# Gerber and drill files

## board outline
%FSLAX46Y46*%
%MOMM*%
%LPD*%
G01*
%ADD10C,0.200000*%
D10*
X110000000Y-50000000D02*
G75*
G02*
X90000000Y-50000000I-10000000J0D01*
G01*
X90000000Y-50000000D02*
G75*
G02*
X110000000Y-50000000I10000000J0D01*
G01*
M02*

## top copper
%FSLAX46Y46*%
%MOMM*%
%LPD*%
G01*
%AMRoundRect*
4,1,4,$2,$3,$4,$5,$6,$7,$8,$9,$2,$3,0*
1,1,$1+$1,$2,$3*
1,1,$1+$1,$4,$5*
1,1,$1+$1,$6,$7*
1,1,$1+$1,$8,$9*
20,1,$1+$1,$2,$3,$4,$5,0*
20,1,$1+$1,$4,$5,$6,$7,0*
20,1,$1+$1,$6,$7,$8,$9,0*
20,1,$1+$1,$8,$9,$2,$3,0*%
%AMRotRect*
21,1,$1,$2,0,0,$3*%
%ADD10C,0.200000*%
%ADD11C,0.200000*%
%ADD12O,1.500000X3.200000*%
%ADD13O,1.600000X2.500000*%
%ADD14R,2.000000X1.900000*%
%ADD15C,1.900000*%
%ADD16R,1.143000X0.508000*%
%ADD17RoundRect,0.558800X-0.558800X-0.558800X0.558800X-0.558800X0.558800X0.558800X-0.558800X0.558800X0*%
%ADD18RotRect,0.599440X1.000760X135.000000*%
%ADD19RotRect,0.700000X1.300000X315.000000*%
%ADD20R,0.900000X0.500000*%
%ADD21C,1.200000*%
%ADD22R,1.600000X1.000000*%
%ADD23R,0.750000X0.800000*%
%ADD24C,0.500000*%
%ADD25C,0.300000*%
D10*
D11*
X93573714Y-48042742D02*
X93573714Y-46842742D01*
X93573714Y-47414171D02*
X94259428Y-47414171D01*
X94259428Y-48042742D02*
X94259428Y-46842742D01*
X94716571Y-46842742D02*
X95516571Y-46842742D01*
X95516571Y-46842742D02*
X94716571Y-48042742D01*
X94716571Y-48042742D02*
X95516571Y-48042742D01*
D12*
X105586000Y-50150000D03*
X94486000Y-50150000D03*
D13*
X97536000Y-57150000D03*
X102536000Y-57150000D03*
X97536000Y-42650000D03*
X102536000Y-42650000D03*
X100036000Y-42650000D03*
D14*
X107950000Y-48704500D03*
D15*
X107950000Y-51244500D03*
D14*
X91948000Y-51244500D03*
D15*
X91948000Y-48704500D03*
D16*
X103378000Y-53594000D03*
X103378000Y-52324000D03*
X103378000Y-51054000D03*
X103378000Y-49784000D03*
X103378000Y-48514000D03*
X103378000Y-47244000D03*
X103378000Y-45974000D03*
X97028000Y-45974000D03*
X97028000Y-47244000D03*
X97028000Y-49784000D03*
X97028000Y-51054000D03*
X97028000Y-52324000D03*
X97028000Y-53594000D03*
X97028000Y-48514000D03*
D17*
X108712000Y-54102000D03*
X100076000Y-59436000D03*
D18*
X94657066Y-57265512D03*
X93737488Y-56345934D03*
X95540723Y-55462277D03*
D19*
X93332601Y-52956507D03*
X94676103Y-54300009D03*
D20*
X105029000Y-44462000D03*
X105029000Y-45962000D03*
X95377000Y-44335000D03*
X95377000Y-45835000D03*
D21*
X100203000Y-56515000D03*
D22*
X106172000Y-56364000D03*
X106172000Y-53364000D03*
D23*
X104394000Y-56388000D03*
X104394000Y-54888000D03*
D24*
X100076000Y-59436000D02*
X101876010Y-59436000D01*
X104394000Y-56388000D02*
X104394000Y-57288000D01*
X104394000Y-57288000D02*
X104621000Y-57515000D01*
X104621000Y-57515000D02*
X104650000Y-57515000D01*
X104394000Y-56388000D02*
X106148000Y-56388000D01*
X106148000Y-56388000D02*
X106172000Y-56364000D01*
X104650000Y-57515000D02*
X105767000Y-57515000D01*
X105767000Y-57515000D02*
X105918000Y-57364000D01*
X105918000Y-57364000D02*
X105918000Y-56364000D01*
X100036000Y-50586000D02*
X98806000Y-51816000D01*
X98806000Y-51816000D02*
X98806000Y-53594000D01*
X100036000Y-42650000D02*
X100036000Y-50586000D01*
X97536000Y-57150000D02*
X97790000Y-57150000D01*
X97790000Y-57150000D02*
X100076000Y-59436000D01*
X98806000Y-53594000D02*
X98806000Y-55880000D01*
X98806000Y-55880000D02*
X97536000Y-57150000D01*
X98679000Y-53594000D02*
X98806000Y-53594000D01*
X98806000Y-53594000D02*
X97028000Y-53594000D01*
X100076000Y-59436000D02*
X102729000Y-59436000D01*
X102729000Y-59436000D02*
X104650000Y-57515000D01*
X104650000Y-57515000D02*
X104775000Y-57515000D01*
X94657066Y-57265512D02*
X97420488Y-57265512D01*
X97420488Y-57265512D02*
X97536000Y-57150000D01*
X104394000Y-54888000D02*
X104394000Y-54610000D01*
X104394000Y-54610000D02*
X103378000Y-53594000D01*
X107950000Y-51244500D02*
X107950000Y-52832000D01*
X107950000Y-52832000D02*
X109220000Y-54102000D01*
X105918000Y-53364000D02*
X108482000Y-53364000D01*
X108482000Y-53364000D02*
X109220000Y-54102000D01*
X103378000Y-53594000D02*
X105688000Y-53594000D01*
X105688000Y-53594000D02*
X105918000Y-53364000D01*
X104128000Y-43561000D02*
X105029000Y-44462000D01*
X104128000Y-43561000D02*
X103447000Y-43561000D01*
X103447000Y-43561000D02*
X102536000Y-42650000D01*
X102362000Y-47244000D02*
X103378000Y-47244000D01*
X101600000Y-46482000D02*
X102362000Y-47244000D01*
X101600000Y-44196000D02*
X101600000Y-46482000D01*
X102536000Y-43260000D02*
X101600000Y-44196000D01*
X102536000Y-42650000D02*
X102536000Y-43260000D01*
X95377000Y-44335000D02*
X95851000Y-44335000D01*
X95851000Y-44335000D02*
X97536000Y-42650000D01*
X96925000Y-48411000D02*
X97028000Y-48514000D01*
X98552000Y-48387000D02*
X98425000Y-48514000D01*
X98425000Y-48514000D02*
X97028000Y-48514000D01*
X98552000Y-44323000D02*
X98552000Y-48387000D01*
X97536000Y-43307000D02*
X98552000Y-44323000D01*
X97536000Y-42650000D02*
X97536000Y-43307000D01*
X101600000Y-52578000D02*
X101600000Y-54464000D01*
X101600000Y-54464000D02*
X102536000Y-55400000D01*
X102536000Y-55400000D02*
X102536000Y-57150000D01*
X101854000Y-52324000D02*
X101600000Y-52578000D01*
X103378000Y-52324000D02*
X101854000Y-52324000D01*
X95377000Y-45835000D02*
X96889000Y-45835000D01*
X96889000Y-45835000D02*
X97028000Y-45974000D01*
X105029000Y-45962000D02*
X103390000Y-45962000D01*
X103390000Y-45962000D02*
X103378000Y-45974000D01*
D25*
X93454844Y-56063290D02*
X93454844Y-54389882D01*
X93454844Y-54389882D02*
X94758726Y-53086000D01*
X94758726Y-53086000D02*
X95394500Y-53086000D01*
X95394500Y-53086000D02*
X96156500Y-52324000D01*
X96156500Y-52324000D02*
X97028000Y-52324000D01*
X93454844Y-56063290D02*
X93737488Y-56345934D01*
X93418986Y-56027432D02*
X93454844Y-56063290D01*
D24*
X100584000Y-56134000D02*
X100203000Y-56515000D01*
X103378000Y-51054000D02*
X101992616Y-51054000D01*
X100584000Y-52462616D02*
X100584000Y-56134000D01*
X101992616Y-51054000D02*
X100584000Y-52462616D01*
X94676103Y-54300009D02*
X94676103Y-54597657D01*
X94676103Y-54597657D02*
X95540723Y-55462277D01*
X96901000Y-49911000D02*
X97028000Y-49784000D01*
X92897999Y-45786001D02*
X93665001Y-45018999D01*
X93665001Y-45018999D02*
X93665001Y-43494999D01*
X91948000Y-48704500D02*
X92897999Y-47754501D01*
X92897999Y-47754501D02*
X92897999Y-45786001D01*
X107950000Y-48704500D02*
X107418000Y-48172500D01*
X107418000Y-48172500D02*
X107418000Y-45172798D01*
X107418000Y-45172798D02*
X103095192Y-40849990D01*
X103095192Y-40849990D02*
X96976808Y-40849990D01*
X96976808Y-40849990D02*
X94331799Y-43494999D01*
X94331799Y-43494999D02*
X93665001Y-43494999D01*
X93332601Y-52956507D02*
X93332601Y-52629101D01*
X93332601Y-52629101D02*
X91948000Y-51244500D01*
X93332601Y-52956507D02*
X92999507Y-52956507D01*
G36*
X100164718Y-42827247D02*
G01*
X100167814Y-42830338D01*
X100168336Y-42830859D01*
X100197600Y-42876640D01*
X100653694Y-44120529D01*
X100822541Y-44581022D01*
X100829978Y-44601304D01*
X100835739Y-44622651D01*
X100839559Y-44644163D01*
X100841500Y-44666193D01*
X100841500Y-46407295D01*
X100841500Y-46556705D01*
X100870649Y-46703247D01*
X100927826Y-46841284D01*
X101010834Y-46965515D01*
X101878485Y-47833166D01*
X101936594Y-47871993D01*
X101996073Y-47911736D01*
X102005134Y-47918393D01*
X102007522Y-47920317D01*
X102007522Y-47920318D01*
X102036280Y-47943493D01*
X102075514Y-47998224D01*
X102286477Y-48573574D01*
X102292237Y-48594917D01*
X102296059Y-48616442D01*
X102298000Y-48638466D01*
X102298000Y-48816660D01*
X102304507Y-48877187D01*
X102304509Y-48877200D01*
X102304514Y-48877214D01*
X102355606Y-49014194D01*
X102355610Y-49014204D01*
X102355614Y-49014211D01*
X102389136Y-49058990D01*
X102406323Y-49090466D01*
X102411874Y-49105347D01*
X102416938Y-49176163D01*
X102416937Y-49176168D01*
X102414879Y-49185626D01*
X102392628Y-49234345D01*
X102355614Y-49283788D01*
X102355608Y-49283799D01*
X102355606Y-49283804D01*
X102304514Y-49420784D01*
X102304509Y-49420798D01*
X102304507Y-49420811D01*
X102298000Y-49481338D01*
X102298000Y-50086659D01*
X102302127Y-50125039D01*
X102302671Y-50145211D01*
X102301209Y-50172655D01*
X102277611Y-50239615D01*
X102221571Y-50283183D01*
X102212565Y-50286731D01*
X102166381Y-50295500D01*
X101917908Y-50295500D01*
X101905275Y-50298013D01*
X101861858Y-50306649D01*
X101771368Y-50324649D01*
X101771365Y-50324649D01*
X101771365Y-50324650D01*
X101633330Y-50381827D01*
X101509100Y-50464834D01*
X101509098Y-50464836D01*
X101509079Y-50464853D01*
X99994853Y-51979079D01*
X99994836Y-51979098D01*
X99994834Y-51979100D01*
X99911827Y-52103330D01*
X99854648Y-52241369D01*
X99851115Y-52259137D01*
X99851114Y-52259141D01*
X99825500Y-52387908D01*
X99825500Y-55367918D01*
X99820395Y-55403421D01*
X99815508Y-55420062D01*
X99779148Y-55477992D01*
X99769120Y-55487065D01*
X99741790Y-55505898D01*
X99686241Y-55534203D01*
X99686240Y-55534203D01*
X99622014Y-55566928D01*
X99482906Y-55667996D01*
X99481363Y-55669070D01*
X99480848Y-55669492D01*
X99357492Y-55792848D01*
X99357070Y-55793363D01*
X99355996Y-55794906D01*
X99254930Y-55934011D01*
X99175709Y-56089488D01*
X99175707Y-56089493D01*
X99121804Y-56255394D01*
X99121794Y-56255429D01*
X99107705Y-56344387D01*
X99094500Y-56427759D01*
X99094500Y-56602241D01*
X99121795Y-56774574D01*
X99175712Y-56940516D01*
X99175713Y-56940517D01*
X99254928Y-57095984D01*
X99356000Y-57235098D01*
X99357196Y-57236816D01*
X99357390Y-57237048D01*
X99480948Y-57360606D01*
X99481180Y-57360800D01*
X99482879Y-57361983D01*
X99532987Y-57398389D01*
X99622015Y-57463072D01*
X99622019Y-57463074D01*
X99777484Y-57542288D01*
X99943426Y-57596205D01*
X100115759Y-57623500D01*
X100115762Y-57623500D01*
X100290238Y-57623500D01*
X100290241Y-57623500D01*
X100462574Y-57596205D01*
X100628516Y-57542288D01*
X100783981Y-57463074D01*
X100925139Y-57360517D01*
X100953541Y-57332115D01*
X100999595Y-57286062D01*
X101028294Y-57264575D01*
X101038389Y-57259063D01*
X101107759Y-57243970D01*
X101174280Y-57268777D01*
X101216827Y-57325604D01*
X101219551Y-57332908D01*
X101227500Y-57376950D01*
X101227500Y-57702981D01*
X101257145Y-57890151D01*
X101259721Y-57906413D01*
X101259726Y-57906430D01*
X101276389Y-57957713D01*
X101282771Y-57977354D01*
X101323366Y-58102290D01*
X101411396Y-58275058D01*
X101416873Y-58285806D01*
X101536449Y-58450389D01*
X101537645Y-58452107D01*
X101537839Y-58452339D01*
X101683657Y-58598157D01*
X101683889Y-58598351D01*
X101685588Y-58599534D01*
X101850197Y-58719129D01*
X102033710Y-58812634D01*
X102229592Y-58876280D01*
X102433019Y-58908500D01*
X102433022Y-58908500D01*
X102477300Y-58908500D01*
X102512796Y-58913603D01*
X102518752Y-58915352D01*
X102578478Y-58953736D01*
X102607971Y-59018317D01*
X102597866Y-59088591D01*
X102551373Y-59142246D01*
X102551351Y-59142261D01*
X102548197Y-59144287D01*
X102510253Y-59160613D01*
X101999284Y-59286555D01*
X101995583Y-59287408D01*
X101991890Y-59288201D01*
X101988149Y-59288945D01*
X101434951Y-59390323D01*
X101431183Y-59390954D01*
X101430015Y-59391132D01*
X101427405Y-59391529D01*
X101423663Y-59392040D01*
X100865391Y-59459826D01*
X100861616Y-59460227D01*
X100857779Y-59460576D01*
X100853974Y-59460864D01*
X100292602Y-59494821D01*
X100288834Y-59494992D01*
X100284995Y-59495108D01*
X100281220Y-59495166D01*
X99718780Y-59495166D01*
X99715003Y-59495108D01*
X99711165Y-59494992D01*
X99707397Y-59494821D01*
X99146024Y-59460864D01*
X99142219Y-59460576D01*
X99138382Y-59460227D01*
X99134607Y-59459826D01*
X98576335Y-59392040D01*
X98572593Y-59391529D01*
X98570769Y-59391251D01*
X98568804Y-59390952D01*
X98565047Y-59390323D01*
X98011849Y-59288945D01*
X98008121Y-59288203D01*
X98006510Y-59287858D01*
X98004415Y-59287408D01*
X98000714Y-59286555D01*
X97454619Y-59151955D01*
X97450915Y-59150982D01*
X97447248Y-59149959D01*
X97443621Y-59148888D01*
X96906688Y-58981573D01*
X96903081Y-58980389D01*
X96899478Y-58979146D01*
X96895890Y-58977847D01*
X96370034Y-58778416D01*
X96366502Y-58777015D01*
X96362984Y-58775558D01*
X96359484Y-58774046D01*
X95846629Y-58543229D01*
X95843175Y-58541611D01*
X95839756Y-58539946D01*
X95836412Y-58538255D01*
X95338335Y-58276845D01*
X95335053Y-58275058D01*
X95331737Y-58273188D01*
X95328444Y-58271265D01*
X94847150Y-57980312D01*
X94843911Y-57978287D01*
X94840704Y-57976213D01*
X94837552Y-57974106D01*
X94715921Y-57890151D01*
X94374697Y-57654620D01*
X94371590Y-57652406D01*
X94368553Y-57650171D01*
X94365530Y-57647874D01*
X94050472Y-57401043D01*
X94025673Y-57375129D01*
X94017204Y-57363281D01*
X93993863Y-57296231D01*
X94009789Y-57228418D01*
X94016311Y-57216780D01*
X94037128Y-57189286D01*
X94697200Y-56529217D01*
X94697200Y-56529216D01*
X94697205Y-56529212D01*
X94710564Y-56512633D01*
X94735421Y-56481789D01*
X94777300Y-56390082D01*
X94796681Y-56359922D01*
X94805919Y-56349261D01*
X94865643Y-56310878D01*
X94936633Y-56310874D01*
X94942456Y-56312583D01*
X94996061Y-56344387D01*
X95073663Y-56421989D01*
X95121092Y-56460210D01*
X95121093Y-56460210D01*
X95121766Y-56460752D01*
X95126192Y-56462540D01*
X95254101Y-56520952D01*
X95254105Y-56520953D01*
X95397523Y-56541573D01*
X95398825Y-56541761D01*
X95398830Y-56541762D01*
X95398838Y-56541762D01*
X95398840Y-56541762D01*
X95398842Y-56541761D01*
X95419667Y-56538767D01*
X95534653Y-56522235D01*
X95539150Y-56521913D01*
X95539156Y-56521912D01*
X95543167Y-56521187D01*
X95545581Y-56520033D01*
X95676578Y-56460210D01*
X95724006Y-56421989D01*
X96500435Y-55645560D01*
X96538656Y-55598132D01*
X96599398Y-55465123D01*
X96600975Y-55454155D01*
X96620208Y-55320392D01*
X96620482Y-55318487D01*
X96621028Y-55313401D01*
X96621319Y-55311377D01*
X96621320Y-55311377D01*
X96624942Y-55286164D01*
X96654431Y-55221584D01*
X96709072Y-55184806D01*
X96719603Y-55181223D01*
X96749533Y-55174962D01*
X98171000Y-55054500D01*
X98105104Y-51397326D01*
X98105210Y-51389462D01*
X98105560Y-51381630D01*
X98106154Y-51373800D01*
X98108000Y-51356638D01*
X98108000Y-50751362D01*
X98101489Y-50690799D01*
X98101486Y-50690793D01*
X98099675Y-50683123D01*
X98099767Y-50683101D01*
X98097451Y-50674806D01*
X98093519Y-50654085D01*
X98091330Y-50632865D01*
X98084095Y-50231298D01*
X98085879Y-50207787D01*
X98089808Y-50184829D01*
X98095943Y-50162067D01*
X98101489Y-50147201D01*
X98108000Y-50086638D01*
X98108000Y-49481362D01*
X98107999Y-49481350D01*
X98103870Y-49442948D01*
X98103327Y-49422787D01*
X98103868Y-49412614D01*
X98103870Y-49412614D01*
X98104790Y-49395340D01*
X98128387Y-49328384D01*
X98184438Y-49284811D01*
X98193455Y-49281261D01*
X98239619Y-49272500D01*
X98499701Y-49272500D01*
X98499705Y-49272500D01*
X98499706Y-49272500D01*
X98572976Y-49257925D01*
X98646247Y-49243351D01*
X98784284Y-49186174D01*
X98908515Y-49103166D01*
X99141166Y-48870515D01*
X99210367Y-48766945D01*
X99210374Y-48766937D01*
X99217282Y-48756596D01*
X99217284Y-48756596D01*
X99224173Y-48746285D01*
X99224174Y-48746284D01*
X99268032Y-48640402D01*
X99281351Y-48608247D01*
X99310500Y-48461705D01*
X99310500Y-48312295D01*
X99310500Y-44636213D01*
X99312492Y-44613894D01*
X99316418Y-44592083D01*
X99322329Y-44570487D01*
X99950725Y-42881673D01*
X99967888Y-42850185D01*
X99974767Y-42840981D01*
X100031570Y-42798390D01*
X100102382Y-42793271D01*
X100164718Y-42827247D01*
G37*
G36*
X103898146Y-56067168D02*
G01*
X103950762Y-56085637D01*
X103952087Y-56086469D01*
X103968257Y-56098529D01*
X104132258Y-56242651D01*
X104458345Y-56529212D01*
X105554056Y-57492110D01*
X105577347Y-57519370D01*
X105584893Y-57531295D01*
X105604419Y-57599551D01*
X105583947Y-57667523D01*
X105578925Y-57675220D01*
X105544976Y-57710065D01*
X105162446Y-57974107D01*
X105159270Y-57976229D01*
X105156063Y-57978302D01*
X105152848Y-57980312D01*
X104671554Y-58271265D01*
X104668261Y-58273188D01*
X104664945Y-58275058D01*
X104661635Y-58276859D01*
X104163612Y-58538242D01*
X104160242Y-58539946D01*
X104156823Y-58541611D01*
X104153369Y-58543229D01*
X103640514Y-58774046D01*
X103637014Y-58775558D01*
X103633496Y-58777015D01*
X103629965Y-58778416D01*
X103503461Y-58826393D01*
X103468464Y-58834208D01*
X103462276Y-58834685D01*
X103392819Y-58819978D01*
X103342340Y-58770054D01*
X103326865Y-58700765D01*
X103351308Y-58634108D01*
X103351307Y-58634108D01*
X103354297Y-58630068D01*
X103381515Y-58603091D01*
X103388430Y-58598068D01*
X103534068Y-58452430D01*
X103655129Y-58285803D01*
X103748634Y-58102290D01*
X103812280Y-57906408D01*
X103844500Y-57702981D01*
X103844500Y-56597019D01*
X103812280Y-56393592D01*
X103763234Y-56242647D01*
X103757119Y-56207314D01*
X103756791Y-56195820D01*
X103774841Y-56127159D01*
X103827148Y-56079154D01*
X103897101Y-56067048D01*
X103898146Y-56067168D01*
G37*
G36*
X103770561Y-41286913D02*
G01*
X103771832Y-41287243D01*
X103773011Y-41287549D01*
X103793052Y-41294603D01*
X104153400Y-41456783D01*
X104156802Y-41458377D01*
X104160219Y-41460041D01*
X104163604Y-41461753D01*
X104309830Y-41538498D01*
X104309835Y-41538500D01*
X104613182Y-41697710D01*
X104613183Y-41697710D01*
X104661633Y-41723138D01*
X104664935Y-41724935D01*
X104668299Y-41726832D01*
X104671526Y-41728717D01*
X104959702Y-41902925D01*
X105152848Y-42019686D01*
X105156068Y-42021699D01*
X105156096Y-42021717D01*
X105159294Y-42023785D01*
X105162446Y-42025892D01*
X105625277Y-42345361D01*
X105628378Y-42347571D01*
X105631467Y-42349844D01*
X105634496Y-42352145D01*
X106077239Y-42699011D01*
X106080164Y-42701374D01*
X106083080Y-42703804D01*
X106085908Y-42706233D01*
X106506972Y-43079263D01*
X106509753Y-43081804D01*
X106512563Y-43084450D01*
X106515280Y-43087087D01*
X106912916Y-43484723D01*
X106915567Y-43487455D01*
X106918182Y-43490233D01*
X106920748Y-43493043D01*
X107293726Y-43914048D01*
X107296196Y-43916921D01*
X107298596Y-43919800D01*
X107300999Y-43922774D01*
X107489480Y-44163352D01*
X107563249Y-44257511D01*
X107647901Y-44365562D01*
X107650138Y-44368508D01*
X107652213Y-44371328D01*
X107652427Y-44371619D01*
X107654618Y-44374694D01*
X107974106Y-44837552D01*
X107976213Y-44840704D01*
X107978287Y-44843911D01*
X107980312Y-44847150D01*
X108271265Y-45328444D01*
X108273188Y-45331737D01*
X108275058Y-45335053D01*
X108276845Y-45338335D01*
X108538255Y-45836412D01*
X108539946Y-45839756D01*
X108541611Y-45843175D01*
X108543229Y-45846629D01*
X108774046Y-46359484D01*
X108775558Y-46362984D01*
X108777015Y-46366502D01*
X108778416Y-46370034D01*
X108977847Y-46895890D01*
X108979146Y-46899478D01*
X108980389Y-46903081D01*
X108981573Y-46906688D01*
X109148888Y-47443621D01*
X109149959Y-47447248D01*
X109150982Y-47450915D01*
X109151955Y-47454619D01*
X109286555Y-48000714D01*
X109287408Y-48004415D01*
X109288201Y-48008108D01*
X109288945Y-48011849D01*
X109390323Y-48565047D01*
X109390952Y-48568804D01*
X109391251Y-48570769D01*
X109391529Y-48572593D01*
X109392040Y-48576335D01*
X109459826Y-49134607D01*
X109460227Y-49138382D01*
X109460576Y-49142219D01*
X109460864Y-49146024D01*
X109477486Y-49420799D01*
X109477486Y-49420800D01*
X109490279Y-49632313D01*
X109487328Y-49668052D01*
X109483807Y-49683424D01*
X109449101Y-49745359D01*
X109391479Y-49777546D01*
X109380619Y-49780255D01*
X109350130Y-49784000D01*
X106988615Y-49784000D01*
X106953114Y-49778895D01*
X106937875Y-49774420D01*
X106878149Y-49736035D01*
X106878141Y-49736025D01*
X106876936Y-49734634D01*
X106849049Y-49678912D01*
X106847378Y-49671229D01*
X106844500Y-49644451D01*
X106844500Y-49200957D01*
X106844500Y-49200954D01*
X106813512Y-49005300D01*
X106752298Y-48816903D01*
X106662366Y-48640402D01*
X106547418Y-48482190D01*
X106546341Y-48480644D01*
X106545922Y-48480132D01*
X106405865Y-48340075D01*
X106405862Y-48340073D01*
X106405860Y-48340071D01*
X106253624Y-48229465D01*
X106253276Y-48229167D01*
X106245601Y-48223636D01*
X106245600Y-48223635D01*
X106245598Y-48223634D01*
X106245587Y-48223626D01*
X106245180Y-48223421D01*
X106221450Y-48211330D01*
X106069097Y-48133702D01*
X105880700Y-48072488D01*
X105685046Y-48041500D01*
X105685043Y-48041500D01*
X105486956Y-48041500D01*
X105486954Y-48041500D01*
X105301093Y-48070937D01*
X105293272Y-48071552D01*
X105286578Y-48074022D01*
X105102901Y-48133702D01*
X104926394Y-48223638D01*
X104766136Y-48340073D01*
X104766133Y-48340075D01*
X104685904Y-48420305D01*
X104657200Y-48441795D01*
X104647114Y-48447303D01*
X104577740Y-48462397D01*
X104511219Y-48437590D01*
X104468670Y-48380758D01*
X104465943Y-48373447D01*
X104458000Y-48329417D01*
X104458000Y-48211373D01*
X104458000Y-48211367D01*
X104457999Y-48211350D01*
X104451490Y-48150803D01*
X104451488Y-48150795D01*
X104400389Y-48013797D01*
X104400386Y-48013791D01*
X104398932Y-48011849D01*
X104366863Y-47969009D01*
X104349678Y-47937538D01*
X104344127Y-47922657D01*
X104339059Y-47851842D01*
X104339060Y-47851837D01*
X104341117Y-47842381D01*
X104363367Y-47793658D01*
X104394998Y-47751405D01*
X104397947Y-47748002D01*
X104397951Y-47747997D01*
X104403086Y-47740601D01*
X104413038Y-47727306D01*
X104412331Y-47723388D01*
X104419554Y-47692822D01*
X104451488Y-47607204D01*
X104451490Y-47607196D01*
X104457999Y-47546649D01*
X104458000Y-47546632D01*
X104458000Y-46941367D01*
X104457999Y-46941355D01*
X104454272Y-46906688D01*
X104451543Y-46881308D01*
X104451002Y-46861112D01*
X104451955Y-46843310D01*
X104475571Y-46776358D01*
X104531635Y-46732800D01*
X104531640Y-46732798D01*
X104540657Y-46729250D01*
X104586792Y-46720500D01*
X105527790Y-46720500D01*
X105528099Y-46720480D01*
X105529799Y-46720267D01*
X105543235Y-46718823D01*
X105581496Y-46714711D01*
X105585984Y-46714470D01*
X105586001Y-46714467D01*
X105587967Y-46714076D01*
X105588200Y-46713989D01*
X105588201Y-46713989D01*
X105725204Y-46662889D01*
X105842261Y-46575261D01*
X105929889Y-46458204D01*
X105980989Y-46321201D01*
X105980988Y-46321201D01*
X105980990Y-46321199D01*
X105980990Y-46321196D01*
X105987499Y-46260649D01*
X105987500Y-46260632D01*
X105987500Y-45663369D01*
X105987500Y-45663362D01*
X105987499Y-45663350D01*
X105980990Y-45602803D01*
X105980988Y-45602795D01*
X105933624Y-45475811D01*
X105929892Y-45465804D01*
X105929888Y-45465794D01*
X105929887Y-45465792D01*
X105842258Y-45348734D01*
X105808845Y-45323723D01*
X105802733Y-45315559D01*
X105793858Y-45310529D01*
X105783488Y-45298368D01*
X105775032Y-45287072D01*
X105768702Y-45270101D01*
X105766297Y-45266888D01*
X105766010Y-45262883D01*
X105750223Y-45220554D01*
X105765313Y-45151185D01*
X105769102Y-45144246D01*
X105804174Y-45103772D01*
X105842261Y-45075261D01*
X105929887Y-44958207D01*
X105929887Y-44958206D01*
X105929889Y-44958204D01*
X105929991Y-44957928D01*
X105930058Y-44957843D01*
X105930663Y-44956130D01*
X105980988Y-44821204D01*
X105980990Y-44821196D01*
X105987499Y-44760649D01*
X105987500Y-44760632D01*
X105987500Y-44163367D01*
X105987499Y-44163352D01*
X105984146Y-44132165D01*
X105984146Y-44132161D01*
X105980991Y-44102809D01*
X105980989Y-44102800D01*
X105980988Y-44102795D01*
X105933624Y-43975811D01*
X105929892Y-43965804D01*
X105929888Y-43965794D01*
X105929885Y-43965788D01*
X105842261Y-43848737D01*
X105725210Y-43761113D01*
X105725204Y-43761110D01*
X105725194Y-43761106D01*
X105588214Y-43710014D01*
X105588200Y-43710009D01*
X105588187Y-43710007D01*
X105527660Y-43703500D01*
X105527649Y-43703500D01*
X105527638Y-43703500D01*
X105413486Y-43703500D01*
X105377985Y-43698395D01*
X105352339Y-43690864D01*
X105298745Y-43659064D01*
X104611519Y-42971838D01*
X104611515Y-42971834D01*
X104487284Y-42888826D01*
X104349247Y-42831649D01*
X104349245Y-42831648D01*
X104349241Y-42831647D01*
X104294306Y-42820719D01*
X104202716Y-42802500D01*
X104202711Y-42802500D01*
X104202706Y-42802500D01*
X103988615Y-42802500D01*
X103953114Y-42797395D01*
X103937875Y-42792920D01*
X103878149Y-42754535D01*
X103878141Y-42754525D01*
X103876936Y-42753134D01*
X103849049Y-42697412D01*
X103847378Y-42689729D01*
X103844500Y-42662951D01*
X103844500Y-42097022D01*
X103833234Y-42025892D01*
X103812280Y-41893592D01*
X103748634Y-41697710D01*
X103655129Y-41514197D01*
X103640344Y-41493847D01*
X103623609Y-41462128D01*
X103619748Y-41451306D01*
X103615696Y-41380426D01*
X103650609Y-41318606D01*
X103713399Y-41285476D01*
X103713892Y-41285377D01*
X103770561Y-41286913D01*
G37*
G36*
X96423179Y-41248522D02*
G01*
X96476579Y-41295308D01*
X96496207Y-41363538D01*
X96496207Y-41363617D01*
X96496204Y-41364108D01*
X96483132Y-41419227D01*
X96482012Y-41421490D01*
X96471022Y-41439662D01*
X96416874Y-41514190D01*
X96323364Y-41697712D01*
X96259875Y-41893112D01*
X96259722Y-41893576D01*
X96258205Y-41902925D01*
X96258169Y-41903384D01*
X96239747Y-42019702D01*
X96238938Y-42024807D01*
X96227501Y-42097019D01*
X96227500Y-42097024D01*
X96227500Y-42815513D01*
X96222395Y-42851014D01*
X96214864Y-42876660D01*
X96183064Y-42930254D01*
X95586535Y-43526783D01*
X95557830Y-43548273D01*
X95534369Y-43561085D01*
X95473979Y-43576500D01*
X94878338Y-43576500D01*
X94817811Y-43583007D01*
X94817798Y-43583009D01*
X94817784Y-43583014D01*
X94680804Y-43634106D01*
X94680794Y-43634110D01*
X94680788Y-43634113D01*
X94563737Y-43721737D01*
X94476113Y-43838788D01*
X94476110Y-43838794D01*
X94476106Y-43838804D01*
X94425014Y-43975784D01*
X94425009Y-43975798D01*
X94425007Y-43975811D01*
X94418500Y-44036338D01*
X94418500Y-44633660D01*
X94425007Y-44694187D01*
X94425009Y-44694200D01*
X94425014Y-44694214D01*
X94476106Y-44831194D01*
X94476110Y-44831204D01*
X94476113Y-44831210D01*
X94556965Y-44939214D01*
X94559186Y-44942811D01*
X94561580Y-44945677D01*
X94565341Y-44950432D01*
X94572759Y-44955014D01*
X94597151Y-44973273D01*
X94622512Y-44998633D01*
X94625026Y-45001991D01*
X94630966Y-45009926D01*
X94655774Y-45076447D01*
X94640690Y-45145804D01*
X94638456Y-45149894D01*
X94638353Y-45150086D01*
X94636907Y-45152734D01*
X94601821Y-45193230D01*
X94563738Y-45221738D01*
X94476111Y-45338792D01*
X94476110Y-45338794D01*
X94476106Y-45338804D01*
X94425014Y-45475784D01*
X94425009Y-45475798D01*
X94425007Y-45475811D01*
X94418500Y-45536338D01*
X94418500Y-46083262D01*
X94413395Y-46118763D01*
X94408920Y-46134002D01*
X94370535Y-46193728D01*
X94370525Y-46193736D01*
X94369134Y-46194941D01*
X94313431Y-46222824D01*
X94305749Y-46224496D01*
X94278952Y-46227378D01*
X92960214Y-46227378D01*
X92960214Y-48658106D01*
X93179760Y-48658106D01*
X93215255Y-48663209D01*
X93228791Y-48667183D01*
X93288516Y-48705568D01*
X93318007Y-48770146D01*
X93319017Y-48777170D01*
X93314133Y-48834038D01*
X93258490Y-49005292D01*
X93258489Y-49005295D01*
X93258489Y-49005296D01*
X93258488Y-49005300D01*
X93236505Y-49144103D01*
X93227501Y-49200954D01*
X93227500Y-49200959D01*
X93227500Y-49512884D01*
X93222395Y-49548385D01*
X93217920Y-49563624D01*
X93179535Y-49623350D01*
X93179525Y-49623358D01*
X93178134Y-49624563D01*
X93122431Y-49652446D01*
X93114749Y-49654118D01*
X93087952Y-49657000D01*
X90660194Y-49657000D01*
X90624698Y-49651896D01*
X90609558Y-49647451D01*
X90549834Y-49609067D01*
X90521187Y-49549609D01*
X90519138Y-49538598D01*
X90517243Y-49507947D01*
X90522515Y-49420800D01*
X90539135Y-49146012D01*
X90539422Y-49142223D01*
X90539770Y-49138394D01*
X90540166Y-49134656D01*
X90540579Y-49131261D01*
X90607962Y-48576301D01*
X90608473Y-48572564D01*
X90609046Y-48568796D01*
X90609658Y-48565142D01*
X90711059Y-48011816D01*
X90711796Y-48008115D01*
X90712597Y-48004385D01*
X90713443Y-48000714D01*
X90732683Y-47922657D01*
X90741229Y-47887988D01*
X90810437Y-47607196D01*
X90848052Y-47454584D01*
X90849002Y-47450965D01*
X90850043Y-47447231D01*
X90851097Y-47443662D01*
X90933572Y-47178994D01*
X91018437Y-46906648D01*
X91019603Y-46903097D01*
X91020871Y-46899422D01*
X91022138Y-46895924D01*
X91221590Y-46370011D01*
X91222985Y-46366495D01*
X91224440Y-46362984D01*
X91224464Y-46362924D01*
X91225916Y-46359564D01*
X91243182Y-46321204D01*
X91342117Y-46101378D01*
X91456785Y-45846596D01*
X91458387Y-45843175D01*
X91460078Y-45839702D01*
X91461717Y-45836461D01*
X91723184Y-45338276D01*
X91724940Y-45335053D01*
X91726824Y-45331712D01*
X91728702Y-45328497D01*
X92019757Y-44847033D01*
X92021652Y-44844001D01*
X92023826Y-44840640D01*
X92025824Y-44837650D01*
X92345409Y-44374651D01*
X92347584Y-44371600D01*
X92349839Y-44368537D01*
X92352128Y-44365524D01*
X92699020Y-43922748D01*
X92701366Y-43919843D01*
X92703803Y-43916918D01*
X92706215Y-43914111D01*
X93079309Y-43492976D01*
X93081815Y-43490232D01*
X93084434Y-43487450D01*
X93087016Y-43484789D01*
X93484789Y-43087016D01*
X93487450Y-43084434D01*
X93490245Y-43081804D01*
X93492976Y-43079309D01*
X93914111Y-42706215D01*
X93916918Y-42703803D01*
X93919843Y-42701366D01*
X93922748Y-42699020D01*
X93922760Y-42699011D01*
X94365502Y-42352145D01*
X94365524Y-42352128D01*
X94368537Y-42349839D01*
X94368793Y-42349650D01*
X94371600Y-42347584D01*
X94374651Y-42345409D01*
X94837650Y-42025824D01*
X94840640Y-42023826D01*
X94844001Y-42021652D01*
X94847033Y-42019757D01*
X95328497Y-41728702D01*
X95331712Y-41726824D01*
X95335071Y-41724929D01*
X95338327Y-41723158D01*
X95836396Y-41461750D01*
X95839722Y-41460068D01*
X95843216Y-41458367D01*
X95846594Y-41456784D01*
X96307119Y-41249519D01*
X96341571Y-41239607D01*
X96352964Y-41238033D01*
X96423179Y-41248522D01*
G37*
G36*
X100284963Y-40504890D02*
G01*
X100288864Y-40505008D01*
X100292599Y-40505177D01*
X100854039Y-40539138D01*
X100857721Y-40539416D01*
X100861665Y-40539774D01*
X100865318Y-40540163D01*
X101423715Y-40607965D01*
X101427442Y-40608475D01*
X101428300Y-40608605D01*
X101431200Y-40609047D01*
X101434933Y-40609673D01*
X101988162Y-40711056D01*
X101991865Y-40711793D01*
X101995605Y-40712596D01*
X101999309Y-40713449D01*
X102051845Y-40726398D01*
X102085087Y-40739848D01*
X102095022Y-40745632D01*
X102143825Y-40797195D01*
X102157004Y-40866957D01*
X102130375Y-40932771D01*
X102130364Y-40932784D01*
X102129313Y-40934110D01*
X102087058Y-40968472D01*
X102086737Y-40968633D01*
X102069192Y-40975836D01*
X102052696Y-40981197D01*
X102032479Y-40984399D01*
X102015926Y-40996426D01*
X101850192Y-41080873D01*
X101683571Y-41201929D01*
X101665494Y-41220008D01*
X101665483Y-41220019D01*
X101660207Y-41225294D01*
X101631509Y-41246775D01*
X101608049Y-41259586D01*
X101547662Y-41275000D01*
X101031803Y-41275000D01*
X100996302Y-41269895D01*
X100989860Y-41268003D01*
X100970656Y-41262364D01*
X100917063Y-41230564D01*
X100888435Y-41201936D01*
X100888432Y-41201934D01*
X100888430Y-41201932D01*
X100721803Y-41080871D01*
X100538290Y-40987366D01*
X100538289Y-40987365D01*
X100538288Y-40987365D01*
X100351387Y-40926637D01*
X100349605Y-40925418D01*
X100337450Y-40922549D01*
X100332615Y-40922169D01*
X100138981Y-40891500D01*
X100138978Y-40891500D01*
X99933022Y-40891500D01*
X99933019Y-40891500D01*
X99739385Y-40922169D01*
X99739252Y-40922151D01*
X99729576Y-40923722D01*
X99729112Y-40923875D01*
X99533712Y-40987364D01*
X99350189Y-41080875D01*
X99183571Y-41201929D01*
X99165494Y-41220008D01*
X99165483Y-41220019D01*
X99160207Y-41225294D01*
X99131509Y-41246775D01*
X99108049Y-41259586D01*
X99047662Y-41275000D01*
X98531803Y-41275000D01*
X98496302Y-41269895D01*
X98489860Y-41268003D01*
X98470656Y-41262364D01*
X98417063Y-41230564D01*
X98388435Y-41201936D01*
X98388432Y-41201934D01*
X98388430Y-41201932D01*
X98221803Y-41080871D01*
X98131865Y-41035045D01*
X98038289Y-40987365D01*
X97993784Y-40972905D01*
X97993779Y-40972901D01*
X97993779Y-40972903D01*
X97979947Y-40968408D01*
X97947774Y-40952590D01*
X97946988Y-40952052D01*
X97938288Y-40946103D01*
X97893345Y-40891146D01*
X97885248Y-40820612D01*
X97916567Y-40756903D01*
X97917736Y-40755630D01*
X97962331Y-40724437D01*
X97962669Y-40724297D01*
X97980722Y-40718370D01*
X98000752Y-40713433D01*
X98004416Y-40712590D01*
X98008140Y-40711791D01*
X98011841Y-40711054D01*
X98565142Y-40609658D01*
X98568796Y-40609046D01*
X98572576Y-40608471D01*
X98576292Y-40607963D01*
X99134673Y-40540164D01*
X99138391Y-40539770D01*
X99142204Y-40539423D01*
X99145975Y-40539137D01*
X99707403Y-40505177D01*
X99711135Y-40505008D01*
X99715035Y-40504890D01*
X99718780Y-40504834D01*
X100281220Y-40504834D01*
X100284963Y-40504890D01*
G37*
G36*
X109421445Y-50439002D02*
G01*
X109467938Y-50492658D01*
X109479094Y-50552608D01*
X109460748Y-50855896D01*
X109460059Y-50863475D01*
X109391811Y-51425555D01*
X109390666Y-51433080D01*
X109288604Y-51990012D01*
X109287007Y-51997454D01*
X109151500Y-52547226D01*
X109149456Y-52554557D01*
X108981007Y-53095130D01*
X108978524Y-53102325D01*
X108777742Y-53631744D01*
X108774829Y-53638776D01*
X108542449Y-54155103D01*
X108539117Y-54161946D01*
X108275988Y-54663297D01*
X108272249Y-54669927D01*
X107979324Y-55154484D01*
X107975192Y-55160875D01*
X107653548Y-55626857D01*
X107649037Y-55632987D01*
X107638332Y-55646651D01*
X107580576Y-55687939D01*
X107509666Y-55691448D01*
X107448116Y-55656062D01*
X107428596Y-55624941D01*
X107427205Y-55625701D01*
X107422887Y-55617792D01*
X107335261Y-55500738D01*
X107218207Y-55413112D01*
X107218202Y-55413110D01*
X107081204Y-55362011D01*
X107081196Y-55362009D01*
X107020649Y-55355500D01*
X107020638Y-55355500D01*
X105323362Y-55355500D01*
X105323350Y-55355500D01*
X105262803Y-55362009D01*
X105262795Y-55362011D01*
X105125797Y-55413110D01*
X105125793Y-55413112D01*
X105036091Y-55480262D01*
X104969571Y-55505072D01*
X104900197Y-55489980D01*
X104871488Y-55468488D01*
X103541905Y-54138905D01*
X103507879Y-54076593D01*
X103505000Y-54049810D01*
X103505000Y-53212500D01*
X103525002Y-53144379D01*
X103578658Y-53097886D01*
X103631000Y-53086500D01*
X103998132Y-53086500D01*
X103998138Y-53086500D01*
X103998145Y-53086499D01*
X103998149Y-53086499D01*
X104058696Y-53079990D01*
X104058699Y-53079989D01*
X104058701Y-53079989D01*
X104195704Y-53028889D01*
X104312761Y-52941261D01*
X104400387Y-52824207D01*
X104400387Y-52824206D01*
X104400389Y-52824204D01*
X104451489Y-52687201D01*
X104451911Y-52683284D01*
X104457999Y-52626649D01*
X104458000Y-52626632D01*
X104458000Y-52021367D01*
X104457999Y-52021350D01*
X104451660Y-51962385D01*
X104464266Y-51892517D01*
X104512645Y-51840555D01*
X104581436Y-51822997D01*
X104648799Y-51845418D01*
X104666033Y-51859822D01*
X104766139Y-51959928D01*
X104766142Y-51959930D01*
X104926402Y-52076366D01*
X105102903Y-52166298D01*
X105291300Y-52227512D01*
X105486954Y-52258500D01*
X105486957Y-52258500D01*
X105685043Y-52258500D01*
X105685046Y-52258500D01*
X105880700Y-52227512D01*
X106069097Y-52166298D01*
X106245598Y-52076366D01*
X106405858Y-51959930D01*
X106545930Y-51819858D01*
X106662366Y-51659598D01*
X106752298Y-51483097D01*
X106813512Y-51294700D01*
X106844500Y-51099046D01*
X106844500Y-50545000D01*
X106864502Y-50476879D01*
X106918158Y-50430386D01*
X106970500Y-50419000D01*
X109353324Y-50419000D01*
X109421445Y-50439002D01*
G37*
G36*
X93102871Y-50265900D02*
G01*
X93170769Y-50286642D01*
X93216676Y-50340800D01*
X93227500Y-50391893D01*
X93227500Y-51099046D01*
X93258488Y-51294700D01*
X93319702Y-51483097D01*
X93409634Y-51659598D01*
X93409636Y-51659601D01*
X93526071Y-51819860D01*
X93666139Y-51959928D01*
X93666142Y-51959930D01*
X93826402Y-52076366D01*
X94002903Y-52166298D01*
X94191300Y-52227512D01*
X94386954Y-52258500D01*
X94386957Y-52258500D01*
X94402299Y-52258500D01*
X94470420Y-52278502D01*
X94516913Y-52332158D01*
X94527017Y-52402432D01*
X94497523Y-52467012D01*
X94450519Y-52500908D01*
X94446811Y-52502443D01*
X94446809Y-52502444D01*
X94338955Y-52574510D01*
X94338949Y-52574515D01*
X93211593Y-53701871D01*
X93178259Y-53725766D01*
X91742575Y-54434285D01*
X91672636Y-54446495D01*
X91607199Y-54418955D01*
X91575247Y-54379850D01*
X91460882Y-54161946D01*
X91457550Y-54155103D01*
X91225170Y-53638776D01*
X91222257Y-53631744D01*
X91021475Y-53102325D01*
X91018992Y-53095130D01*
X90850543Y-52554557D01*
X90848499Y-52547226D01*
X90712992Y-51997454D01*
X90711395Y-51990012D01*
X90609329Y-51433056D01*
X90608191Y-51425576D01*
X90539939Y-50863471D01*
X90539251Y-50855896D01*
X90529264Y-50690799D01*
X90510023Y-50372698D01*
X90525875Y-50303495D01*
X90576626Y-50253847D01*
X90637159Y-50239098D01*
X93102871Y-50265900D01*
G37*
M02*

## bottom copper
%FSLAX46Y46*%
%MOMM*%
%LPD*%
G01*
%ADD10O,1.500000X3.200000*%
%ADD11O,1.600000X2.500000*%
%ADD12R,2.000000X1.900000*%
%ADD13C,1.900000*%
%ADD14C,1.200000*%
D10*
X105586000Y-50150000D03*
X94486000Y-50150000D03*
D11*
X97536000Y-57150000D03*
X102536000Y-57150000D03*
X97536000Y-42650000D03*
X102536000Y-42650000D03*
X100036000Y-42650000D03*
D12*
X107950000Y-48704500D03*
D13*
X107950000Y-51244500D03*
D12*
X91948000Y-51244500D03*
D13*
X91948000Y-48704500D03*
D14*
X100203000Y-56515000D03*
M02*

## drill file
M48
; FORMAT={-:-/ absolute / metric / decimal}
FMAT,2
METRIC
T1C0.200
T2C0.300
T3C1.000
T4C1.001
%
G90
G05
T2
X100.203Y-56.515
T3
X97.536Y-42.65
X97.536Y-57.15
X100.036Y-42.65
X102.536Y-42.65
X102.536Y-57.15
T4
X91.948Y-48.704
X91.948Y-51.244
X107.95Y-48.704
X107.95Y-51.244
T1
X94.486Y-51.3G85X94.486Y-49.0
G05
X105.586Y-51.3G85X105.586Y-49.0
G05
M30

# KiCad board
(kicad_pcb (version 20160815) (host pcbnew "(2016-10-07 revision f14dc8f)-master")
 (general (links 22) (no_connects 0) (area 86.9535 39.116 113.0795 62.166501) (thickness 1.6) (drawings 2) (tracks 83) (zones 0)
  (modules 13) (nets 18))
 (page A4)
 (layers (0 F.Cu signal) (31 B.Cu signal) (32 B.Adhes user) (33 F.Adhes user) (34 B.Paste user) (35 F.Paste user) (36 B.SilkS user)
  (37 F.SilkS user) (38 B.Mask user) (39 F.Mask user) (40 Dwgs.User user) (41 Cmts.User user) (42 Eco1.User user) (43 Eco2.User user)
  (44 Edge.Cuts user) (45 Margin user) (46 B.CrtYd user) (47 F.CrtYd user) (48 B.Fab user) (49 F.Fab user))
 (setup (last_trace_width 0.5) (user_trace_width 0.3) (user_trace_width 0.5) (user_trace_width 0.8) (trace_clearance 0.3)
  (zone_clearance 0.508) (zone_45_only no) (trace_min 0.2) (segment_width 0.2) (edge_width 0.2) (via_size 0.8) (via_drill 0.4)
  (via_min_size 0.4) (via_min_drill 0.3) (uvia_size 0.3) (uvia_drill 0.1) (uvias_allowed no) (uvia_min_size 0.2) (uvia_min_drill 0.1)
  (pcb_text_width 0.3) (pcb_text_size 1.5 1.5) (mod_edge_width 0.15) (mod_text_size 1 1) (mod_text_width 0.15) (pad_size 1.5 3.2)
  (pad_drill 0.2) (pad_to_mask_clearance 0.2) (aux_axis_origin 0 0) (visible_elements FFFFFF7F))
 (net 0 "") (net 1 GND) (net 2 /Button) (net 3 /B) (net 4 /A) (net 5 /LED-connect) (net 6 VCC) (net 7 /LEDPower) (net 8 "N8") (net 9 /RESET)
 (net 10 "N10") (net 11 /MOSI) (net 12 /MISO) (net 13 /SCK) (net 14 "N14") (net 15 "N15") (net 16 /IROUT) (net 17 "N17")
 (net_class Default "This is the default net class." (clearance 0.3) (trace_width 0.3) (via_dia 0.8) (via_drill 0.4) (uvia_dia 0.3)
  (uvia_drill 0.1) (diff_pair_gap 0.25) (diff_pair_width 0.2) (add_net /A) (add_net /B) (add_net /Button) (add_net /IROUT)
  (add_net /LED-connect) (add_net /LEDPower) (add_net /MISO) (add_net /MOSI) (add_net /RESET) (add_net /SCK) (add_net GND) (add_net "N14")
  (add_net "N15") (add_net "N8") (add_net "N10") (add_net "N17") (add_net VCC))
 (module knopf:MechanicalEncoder (layer B.Cu) (at 100.036 50.15 180)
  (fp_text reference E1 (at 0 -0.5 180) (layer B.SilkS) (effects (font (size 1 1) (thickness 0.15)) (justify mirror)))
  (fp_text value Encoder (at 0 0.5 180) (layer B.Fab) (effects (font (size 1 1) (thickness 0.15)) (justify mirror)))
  (pad 6 thru_hole oval (at -5.55 0 180) (size 1.5 3.2) (drill oval 0.2 2.5) (layers *.Cu *.Mask))
  (pad 6 thru_hole oval (at 5.55 0 180) (size 1.5 3.2) (drill oval 0.2 2.5) (layers *.Cu *.Mask))
  (pad 5 thru_hole oval (at 2.5 -7 180) (size 1.6 2.5) (drill 1) (layers *.Cu *.Mask) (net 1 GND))
  (pad 4 thru_hole oval (at -2.5 -7 180) (size 1.6 2.5) (drill 1) (layers *.Cu *.Mask) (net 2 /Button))
  (pad 3 thru_hole oval (at 2.5 7.5 180) (size 1.6 2.5) (drill 1) (layers *.Cu *.Mask) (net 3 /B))
  (pad 1 thru_hole oval (at -2.5 7.5 180) (size 1.6 2.5) (drill 1) (layers *.Cu *.Mask) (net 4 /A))
  (pad 2 thru_hole oval (at 0 7.5 180) (size 1.6 2.5) (drill 1) (layers *.Cu *.Mask) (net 1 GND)))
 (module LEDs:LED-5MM (layer F.Cu) (at 107.95 48.7045 270)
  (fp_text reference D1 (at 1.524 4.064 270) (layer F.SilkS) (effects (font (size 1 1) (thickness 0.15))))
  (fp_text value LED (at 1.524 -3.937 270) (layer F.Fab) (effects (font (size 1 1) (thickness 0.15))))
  (pad 1 thru_hole rect (at 0 0) (size 2 1.9) (drill 1.00076) (layers *.Cu *.Mask F.SilkS) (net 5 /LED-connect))
  (pad 2 thru_hole circle (at 2.54 0 270) (size 1.9 1.9) (drill 1.00076) (layers *.Cu *.Mask F.SilkS) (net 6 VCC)))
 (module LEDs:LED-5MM (layer F.Cu) (at 91.948 51.2445 90)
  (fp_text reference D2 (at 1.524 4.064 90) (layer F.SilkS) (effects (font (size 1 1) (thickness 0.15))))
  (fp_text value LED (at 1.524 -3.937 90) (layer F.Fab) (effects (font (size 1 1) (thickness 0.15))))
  (pad 1 thru_hole rect (at 0 0 180) (size 2 1.9) (drill 1.00076) (layers *.Cu *.Mask F.SilkS) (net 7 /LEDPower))
  (pad 2 thru_hole circle (at 2.54 0 90) (size 1.9 1.9) (drill 1.00076) (layers *.Cu *.Mask F.SilkS) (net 5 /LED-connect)))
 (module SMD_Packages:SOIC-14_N (layer F.Cu) (at 100.076 49.784 90)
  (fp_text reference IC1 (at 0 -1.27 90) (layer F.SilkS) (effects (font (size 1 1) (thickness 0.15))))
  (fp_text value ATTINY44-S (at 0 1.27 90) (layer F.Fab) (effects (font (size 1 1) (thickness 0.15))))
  (pad 1 smd rect (at -3.81 3.302 90) (size 0.508 1.143) (layers F.Cu F.Paste F.Mask) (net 6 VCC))
  (pad 2 smd rect (at -2.54 3.302 90) (size 0.508 1.143) (layers F.Cu F.Paste F.Mask) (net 2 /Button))
  (pad 3 smd rect (at -1.27 3.302 90) (size 0.508 1.143) (layers F.Cu F.Paste F.Mask) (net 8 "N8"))
  (pad 4 smd rect (at 0 3.302 90) (size 0.508 1.143) (layers F.Cu F.Paste F.Mask) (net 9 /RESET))
  (pad 5 smd rect (at 1.27 3.302 90) (size 0.508 1.143) (layers F.Cu F.Paste F.Mask) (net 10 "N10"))
  (pad 6 smd rect (at 2.54 3.302 90) (size 0.508 1.143) (layers F.Cu F.Paste F.Mask) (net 4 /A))
  (pad 7 smd rect (at 3.81 3.302 90) (size 0.508 1.143) (layers F.Cu F.Paste F.Mask) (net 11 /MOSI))
  (pad 8 smd rect (at 3.81 -3.048 90) (size 0.508 1.143) (layers F.Cu F.Paste F.Mask) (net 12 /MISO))
  (pad 9 smd rect (at 2.54 -3.048 90) (size 0.508 1.143) (layers F.Cu F.Paste F.Mask) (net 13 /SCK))
  (pad 11 smd rect (at 0 -3.048 90) (size 0.508 1.143) (layers F.Cu F.Paste F.Mask) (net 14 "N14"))
  (pad 12 smd rect (at -1.27 -3.048 90) (size 0.508 1.143) (layers F.Cu F.Paste F.Mask) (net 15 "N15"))
  (pad 13 smd rect (at -2.54 -3.048 90) (size 0.508 1.143) (layers F.Cu F.Paste F.Mask) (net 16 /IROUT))
  (pad 14 smd rect (at -3.81 -3.048 90) (size 0.508 1.143) (layers F.Cu F.Paste F.Mask) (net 1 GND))
  (pad 10 smd rect (at 1.27 -3.048 90) (size 0.508 1.143) (layers F.Cu F.Paste F.Mask) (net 3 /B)))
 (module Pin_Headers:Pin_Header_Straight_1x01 (layer F.Cu) (at 108.712 54.102)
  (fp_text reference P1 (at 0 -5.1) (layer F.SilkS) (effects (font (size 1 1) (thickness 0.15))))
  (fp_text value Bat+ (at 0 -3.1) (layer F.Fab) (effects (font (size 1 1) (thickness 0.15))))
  (pad 1 smd roundrect (at 0 0) (size 2.2352 2.2352) (layers F.Cu F.Paste F.Mask) (roundrect_rratio 0.25) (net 6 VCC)))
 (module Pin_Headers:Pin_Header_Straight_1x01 (layer F.Cu) (at 100.076 59.436)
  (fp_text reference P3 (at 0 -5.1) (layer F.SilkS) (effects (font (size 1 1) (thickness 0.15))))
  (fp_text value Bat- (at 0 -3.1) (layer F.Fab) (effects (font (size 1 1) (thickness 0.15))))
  (pad 1 smd roundrect (at 0 0) (size 2.2352 2.2352) (layers F.Cu F.Paste F.Mask) (roundrect_rratio 0.25) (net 1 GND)))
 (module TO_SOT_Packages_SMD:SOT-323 (layer F.Cu) (at 94.869 56.134 135)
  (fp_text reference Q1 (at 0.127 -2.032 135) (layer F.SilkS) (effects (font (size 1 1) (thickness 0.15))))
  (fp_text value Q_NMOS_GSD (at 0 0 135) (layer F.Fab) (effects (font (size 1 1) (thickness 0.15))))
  (pad 2 smd rect (at -0.65024 -0.94996 135) (size 0.59944 1.00076) (layers F.Cu F.Paste F.Mask) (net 1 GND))
  (pad 1 smd rect (at 0.65024 -0.94996 135) (size 0.59944 1.00076) (layers F.Cu F.Paste F.Mask) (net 16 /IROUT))
  (pad 3 smd rect (at 0 0.94996 135) (size 0.59944 1.00076) (layers F.Cu F.Paste F.Mask) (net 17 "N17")))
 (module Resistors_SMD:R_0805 (layer F.Cu) (at 94.004352 53.628258 315)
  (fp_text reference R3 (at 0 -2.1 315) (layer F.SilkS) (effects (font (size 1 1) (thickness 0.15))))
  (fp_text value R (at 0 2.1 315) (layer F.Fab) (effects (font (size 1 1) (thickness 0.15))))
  (pad 1 smd rect (at -0.949999 0 315) (size 0.7 1.3) (layers F.Cu F.Paste F.Mask) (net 7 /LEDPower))
  (pad 2 smd rect (at 0.949999 0 315) (size 0.7 1.3) (layers F.Cu F.Paste F.Mask) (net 17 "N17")))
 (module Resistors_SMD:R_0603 (layer F.Cu) (at 105.029 45.212 270)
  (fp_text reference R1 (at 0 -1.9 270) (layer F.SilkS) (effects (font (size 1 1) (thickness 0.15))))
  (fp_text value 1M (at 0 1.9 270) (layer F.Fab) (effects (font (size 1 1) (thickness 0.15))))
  (pad 1 smd rect (at -0.75 0 270) (size 0.5 0.9) (layers F.Cu F.Paste F.Mask) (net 4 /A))
  (pad 2 smd rect (at 0.75 0 270) (size 0.5 0.9) (layers F.Cu F.Paste F.Mask) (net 11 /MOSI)))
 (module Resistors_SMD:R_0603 (layer F.Cu) (at 95.377 45.085 270)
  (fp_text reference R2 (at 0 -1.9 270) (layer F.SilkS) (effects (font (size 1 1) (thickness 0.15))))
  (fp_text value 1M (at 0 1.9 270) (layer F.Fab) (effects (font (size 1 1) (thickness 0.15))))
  (pad 1 smd rect (at -0.75 0 270) (size 0.5 0.9) (layers F.Cu F.Paste F.Mask) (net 3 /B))
  (pad 2 smd rect (at 0.75 0 270) (size 0.5 0.9) (layers F.Cu F.Paste F.Mask) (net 12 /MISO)))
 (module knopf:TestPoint (layer F.Cu) (at 100.203 56.515)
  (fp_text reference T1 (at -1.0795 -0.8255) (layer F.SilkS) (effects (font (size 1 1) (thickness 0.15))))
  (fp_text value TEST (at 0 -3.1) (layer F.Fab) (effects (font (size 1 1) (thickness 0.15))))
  (pad 1 thru_hole circle (at 0 0) (size 1.2 1.2) (drill 0.3) (layers *.Cu *.Mask F.SilkS) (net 8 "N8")))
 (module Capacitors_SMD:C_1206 (layer F.Cu) (at 106.172 54.864 270)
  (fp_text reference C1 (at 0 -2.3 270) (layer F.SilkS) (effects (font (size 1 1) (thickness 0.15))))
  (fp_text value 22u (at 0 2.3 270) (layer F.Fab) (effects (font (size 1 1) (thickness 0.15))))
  (pad 2 smd rect (at 1.5 0 270) (size 1 1.6) (layers F.Cu F.Paste F.Mask) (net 1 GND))
  (pad 1 smd rect (at -1.5 0 270) (size 1 1.6) (layers F.Cu F.Paste F.Mask) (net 6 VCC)))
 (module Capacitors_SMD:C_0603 (layer F.Cu) (at 104.394 55.638 270)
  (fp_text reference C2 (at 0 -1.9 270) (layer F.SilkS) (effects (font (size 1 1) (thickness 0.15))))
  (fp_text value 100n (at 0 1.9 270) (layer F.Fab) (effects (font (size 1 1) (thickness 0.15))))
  (pad 2 smd rect (at 0.75 0 270) (size 0.8 0.75) (layers F.Cu F.Paste F.Mask) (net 1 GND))
  (pad 1 smd rect (at -0.75 0 270) (size 0.8 0.75) (layers F.Cu F.Paste F.Mask) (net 6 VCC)))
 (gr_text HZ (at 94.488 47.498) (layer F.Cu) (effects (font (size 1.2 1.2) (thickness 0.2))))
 (gr_circle (center 100 50) (end 110 50) (layer Edge.Cuts) (width 0.2))
 (segment (start 100.076 59.436) (end 101.87601 59.436) (width 0.5) (layer F.Cu) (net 1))
 (segment (start 104.394 56.388) (end 104.394 57.288) (width 0.5) (layer F.Cu) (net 1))
 (segment (start 104.394 57.288) (end 104.621 57.515) (width 0.5) (layer F.Cu) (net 1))
 (segment (start 104.621 57.515) (end 104.65 57.515) (width 0.5) (layer F.Cu) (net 1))
 (segment (start 104.394 56.388) (end 106.148 56.388) (width 0.5) (layer F.Cu) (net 1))
 (segment (start 106.148 56.388) (end 106.172 56.364) (width 0.5) (layer F.Cu) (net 1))
 (segment (start 104.65 57.515) (end 105.767 57.515) (width 0.5) (layer F.Cu) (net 1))
 (segment (start 105.767 57.515) (end 105.918 57.364) (width 0.5) (layer F.Cu) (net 1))
 (segment (start 105.918 57.364) (end 105.918 56.364) (width 0.5) (layer F.Cu) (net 1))
 (segment (start 100.036 50.586) (end 98.806 51.816) (width 0.5) (layer F.Cu) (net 1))
 (segment (start 98.806 51.816) (end 98.806 53.594) (width 0.5) (layer F.Cu) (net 1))
 (segment (start 100.036 42.65) (end 100.036 50.586) (width 0.5) (layer F.Cu) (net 1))
 (segment (start 97.536 57.15) (end 97.79 57.15) (width 0.5) (layer F.Cu) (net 1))
 (segment (start 97.79 57.15) (end 100.076 59.436) (width 0.5) (layer F.Cu) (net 1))
 (segment (start 98.806 53.594) (end 98.806 55.88) (width 0.5) (layer F.Cu) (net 1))
 (segment (start 98.806 55.88) (end 97.536 57.15) (width 0.5) (layer F.Cu) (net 1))
 (segment (start 98.679 53.594) (end 98.806 53.594) (width 0.5) (layer F.Cu) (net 1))
 (segment (start 98.806 53.594) (end 97.028 53.594) (width 0.5) (layer F.Cu) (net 1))
 (segment (start 100.076 59.436) (end 102.729 59.436) (width 0.5) (layer F.Cu) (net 1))
 (segment (start 102.729 59.436) (end 104.65 57.515) (width 0.5) (layer F.Cu) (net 1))
 (segment (start 104.65 57.515) (end 104.775 57.515) (width 0.5) (layer F.Cu) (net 1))
 (segment (start 94.657066 57.265512) (end 97.420488 57.265512) (width 0.5) (layer F.Cu) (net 1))
 (segment (start 97.420488 57.265512) (end 97.536 57.15) (width 0.5) (layer F.Cu) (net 1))
 (segment (start 104.394 54.888) (end 104.394 54.61) (width 0.5) (layer F.Cu) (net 6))
 (segment (start 104.394 54.61) (end 103.378 53.594) (width 0.5) (layer F.Cu) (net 6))
 (segment (start 107.95 51.2445) (end 107.95 52.832) (width 0.5) (layer F.Cu) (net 6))
 (segment (start 107.95 52.832) (end 109.22 54.102) (width 0.5) (layer F.Cu) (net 6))
 (segment (start 105.918 53.364) (end 108.482 53.364) (width 0.5) (layer F.Cu) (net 6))
 (segment (start 108.482 53.364) (end 109.22 54.102) (width 0.5) (layer F.Cu) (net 6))
 (segment (start 103.378 53.594) (end 105.688 53.594) (width 0.5) (layer F.Cu) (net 6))
 (segment (start 105.688 53.594) (end 105.918 53.364) (width 0.5) (layer F.Cu) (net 6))
 (segment (start 104.128 43.561) (end 105.029 44.462) (width 0.5) (layer F.Cu) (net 4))
 (segment (start 104.128 43.561) (end 103.447 43.561) (width 0.5) (layer F.Cu) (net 4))
 (segment (start 103.447 43.561) (end 102.536 42.65) (width 0.5) (layer F.Cu) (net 4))
 (segment (start 102.362 47.244) (end 103.378 47.244) (width 0.5) (layer F.Cu) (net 4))
 (segment (start 101.6 46.482) (end 102.362 47.244) (width 0.5) (layer F.Cu) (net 4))
 (segment (start 101.6 44.196) (end 101.6 46.482) (width 0.5) (layer F.Cu) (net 4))
 (segment (start 102.536 43.26) (end 101.6 44.196) (width 0.5) (layer F.Cu) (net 4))
 (segment (start 102.536 42.65) (end 102.536 43.26) (width 0.5) (layer F.Cu) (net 4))
 (segment (start 95.377 44.335) (end 95.851 44.335) (width 0.5) (layer F.Cu) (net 3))
 (segment (start 95.851 44.335) (end 97.536 42.65) (width 0.5) (layer F.Cu) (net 3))
 (segment (start 96.925 48.411) (end 97.028 48.514) (width 0.5) (layer F.Cu) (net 3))
 (segment (start 98.552 48.387) (end 98.425 48.514) (width 0.5) (layer F.Cu) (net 3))
 (segment (start 98.425 48.514) (end 97.028 48.514) (width 0.5) (layer F.Cu) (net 3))
 (segment (start 98.552 44.323) (end 98.552 48.387) (width 0.5) (layer F.Cu) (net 3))
 (segment (start 97.536 43.307) (end 98.552 44.323) (width 0.5) (layer F.Cu) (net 3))
 (segment (start 97.536 42.65) (end 97.536 43.307) (width 0.5) (layer F.Cu) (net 3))
 (segment (start 101.6 52.578) (end 101.6 54.464) (width 0.5) (layer F.Cu) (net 2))
 (segment (start 101.6 54.464) (end 102.536 55.4) (width 0.5) (layer F.Cu) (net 2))
 (segment (start 102.536 55.4) (end 102.536 57.15) (width 0.5) (layer F.Cu) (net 2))
 (segment (start 101.854 52.324) (end 101.6 52.578) (width 0.5) (layer F.Cu) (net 2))
 (segment (start 103.378 52.324) (end 101.854 52.324) (width 0.5) (layer F.Cu) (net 2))
 (segment (start 95.377 45.835) (end 96.889 45.835) (width 0.5) (layer F.Cu) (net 12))
 (segment (start 96.889 45.835) (end 97.028 45.974) (width 0.5) (layer F.Cu) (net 12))
 (segment (start 105.029 45.962) (end 103.39 45.962) (width 0.5) (layer F.Cu) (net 11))
 (segment (start 103.39 45.962) (end 103.378 45.974) (width 0.5) (layer F.Cu) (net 11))
 (segment (start 93.454844 56.06329) (end 93.454844 54.389882) (width 0.3) (layer F.Cu) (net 16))
 (segment (start 93.454844 54.389882) (end 94.758726 53.086) (width 0.3) (layer F.Cu) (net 16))
 (segment (start 94.758726 53.086) (end 95.3945 53.086) (width 0.3) (layer F.Cu) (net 16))
 (segment (start 95.3945 53.086) (end 96.1565 52.324) (width 0.3) (layer F.Cu) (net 16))
 (segment (start 96.1565 52.324) (end 97.028 52.324) (width 0.3) (layer F.Cu) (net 16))
 (segment (start 93.454844 56.06329) (end 93.737488 56.345934) (width 0.3) (layer F.Cu) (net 16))
 (segment (start 93.418986 56.027432) (end 93.454844 56.06329) (width 0.3) (layer F.Cu) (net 16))
 (segment (start 100.584 56.134) (end 100.203 56.515) (width 0.5) (layer F.Cu) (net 8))
 (segment (start 103.378 51.054) (end 101.992616 51.054) (width 0.5) (layer F.Cu) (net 8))
 (segment (start 100.584 52.462616) (end 100.584 56.134) (width 0.5) (layer F.Cu) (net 8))
 (segment (start 101.992616 51.054) (end 100.584 52.462616) (width 0.5) (layer F.Cu) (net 8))
 (segment (start 94.676103 54.300009) (end 94.676103 54.597657) (width 0.5) (layer F.Cu) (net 17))
 (segment (start 94.676103 54.597657) (end 95.540723 55.462277) (width 0.5) (layer F.Cu) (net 17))
 (segment (start 96.901 49.911) (end 97.028 49.784) (width 0.5) (layer F.Cu) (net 14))
 (segment (start 92.897999 45.786001) (end 93.665001 45.018999) (width 0.5) (layer F.Cu) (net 5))
 (segment (start 93.665001 45.018999) (end 93.665001 43.494999) (width 0.5) (layer F.Cu) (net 5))
 (segment (start 91.948 48.7045) (end 92.897999 47.754501) (width 0.5) (layer F.Cu) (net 5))
 (segment (start 92.897999 47.754501) (end 92.897999 45.786001) (width 0.5) (layer F.Cu) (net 5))
 (segment (start 107.95 48.7045) (end 107.418 48.1725) (width 0.5) (layer F.Cu) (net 5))
 (segment (start 107.418 48.1725) (end 107.418 45.172798) (width 0.5) (layer F.Cu) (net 5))
 (segment (start 107.418 45.172798) (end 103.095192 40.84999) (width 0.5) (layer F.Cu) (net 5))
 (segment (start 103.095192 40.84999) (end 96.976808 40.84999) (width 0.5) (layer F.Cu) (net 5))
 (segment (start 96.976808 40.84999) (end 94.331799 43.494999) (width 0.5) (layer F.Cu) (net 5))
 (segment (start 94.331799 43.494999) (end 93.665001 43.494999) (width 0.5) (layer F.Cu) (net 5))
 (segment (start 93.332601 52.956507) (end 93.332601 52.629101) (width 0.5) (layer F.Cu) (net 7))
 (segment (start 93.332601 52.629101) (end 91.948 51.2445) (width 0.5) (layer F.Cu) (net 7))
 (segment (start 93.332601 52.956507) (end 92.999507 52.956507) (width 0.5) (layer F.Cu) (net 7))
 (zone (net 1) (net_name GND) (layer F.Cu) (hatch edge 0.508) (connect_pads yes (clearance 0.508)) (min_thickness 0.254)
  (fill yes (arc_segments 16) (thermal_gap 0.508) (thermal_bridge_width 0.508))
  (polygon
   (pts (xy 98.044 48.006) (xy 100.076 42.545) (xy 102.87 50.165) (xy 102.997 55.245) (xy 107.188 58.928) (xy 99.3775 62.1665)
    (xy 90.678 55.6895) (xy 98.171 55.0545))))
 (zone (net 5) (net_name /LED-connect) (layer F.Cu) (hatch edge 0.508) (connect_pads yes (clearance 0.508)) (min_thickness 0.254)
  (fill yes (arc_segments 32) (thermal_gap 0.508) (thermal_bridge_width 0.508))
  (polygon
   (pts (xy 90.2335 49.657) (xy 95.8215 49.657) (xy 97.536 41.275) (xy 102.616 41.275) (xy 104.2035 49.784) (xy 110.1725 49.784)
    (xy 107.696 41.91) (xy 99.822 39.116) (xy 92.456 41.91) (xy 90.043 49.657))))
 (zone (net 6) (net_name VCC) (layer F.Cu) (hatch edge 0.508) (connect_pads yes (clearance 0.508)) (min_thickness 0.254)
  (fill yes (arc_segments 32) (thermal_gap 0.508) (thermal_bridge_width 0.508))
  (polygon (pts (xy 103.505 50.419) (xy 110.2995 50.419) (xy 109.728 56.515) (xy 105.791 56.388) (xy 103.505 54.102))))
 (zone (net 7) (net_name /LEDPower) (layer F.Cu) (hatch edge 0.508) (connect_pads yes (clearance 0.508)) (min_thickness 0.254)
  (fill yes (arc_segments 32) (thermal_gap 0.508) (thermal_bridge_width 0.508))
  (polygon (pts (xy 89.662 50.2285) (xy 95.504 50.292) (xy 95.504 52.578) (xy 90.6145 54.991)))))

